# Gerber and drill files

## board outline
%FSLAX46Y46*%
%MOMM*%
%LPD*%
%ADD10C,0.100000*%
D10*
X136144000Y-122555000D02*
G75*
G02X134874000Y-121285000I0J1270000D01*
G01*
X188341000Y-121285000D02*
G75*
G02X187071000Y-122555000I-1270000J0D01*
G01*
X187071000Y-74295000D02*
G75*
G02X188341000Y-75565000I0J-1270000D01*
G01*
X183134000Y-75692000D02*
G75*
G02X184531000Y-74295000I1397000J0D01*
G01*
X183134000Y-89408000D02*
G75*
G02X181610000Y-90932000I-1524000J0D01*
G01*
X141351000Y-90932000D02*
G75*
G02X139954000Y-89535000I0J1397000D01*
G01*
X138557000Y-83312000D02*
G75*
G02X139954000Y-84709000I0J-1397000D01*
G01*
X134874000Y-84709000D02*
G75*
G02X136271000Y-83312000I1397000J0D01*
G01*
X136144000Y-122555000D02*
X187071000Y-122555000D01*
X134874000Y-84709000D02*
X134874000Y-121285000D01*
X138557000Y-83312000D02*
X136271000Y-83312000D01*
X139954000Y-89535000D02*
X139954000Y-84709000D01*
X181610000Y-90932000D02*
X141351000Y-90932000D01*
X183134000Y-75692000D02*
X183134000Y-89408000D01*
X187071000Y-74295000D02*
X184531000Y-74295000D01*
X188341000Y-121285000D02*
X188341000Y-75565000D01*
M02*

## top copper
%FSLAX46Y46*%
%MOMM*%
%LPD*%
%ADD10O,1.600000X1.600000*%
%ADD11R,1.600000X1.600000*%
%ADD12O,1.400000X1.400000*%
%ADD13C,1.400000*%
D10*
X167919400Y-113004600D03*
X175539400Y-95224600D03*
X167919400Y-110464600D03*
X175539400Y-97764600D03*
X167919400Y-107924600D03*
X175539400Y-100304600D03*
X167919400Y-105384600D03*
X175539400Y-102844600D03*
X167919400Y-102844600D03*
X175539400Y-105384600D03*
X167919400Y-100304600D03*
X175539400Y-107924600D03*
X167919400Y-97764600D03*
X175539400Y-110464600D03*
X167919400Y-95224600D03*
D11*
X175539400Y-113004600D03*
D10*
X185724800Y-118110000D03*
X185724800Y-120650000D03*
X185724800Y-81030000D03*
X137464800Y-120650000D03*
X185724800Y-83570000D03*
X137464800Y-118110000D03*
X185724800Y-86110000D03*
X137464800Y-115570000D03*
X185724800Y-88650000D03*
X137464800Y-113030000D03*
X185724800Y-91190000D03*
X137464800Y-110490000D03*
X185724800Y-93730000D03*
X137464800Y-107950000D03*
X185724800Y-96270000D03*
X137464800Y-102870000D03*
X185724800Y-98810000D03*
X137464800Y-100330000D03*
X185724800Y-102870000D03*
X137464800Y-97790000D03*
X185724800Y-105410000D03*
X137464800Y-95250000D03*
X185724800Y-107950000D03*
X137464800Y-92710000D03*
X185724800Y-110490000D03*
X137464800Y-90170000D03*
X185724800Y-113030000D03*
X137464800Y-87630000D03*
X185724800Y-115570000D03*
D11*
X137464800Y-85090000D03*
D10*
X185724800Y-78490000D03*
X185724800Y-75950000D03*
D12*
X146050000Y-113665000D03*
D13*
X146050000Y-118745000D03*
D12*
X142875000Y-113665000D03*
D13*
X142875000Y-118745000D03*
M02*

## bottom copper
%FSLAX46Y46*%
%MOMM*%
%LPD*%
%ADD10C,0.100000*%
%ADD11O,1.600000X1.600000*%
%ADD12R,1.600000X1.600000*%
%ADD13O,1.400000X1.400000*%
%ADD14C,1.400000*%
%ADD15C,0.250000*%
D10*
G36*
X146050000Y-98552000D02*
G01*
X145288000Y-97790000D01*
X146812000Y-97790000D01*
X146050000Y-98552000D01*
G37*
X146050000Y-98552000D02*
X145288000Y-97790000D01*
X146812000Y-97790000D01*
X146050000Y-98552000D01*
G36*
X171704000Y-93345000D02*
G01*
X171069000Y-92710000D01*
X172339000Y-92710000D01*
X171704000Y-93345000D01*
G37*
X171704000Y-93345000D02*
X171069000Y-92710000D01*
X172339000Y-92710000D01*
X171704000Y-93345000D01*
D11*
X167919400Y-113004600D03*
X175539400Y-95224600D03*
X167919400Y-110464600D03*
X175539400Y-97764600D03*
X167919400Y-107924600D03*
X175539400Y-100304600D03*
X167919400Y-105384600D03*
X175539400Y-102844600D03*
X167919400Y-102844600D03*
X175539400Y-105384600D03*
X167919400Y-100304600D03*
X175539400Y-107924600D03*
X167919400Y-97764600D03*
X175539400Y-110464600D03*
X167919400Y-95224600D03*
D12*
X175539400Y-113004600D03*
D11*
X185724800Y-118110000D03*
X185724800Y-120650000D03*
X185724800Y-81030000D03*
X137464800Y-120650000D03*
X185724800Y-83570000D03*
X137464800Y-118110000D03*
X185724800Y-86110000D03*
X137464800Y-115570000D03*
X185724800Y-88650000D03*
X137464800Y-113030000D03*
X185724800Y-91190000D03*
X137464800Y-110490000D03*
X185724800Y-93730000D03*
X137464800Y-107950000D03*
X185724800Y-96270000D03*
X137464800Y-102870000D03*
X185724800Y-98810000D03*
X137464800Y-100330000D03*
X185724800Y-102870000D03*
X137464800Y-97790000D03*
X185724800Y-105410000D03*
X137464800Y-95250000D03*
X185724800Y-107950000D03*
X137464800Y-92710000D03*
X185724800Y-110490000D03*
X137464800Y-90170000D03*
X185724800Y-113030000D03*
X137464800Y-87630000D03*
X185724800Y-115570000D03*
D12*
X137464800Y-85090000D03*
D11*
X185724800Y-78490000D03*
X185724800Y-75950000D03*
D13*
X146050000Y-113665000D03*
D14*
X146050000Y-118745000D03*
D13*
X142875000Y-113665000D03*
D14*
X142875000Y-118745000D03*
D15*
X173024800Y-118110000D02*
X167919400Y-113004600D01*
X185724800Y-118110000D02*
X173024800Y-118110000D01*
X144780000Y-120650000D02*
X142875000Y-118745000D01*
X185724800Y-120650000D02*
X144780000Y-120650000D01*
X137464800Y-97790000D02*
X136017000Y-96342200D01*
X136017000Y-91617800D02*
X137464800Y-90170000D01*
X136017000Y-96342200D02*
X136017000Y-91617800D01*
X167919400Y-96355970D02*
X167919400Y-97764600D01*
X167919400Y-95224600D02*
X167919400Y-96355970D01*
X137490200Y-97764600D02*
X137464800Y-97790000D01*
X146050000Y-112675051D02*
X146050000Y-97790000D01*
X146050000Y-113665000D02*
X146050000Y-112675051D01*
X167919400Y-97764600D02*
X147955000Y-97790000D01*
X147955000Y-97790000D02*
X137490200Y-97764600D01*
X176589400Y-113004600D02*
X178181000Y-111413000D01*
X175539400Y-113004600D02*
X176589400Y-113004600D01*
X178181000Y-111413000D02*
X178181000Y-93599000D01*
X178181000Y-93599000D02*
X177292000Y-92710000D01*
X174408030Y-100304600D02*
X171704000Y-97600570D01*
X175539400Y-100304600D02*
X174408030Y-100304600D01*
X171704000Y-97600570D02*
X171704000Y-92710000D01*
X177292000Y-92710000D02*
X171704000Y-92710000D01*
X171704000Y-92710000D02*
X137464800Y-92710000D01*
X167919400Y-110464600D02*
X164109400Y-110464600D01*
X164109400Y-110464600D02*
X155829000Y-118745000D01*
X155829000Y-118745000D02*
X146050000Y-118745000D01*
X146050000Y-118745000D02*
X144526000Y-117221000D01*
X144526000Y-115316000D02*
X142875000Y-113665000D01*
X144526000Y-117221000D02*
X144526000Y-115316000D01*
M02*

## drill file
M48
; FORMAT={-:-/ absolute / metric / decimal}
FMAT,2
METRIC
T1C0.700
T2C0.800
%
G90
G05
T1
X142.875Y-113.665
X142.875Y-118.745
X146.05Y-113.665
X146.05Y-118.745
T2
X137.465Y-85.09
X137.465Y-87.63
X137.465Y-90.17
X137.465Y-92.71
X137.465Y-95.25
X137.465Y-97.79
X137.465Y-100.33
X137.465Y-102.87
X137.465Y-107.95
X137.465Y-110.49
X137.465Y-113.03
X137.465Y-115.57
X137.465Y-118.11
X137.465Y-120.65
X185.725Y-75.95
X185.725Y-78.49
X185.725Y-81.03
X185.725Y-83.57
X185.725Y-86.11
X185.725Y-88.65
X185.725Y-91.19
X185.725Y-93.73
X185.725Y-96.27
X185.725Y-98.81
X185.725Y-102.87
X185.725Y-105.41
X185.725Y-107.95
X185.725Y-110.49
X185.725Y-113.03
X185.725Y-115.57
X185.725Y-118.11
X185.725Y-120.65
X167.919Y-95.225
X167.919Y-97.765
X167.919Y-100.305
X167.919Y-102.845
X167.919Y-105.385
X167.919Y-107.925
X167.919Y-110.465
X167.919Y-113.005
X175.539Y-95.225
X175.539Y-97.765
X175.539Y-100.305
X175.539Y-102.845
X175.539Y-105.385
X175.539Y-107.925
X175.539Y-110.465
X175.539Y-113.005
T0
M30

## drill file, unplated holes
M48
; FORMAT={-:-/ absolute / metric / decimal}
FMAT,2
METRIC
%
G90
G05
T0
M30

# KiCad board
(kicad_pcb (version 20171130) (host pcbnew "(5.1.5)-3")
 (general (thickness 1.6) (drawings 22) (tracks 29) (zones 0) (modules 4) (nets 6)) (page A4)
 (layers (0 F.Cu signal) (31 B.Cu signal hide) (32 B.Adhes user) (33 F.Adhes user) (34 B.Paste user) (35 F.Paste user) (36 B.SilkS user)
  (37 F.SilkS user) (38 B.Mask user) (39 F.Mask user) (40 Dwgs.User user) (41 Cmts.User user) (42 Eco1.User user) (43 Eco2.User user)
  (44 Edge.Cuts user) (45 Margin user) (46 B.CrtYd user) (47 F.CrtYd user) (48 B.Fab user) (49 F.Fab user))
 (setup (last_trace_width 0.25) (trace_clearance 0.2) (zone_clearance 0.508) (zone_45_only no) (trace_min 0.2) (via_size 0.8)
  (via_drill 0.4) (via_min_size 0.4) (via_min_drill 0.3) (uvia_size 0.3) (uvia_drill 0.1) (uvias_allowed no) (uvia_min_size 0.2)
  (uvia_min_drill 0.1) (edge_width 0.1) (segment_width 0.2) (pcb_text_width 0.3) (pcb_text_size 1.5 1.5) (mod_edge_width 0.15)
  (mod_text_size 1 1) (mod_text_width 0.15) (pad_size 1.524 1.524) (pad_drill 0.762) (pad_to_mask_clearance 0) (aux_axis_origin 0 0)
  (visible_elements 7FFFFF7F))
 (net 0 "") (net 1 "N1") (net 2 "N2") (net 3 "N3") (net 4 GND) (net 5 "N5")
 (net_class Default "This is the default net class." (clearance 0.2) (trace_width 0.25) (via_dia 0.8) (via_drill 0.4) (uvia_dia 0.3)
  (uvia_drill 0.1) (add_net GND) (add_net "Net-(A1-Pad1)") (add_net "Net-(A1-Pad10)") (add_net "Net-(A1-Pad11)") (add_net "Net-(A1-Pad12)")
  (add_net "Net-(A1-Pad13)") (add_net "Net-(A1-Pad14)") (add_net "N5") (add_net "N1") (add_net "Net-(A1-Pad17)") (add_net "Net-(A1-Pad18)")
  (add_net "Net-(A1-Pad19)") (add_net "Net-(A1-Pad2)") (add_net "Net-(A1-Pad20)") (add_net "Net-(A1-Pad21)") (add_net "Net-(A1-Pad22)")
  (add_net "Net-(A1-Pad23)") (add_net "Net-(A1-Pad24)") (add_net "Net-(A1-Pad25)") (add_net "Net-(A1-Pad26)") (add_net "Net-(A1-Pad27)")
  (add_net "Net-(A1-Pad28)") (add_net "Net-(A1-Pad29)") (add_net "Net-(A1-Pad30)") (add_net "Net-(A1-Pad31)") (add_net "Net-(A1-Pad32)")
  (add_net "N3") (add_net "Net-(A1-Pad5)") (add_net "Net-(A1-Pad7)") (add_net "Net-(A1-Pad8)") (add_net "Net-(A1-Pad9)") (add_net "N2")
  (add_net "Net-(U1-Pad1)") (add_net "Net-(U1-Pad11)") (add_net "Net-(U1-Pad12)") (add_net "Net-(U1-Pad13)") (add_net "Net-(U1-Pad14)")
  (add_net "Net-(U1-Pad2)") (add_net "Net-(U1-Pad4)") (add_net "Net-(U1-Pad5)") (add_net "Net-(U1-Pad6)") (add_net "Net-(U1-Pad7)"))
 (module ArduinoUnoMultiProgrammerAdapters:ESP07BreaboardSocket (layer F.Cu) (at 171.704 102.616)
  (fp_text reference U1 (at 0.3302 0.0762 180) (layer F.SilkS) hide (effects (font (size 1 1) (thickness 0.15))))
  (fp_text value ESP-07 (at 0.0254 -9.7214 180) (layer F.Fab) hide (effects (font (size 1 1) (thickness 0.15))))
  (pad 16 thru_hole oval (at -3.7846 10.3886 180) (size 1.6 1.6) (drill 0.8) (layers *.Cu *.Mask) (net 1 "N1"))
  (pad 1 thru_hole oval (at 3.8354 -7.3914 180) (size 1.6 1.6) (drill 0.8) (layers *.Cu *.Mask))
  (pad 15 thru_hole oval (at -3.7846 7.8486 180) (size 1.6 1.6) (drill 0.8) (layers *.Cu *.Mask) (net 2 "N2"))
  (pad 2 thru_hole oval (at 3.8354 -4.8514 180) (size 1.6 1.6) (drill 0.8) (layers *.Cu *.Mask))
  (pad 14 thru_hole oval (at -3.7846 5.3086 180) (size 1.6 1.6) (drill 0.8) (layers *.Cu *.Mask))
  (pad 3 thru_hole oval (at 3.8354 -2.3114 180) (size 1.6 1.6) (drill 0.8) (layers *.Cu *.Mask) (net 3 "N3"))
  (pad 13 thru_hole oval (at -3.7846 2.7686 180) (size 1.6 1.6) (drill 0.8) (layers *.Cu *.Mask))
  (pad 4 thru_hole oval (at 3.8354 0.2286 180) (size 1.6 1.6) (drill 0.8) (layers *.Cu *.Mask))
  (pad 12 thru_hole oval (at -3.7846 0.2286 180) (size 1.6 1.6) (drill 0.8) (layers *.Cu *.Mask))
  (pad 5 thru_hole oval (at 3.8354 2.7686 180) (size 1.6 1.6) (drill 0.8) (layers *.Cu *.Mask))
  (pad 11 thru_hole oval (at -3.7846 -2.3114 180) (size 1.6 1.6) (drill 0.8) (layers *.Cu *.Mask))
  (pad 6 thru_hole oval (at 3.8354 5.3086 180) (size 1.6 1.6) (drill 0.8) (layers *.Cu *.Mask))
  (pad 10 thru_hole oval (at -3.7846 -4.8514 180) (size 1.6 1.6) (drill 0.8) (layers *.Cu *.Mask) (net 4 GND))
  (pad 7 thru_hole oval (at 3.8354 7.8486 180) (size 1.6 1.6) (drill 0.8) (layers *.Cu *.Mask))
  (pad 9 thru_hole oval (at -3.7846 -7.3914 180) (size 1.6 1.6) (drill 0.8) (layers *.Cu *.Mask) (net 4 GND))
  (pad 8 thru_hole rect (at 3.8354 10.3886 270) (size 1.6 1.6) (drill 0.8) (layers *.Cu *.Mask) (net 3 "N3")))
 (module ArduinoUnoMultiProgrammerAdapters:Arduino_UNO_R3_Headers (layer F.Cu) (at 160.274 89.535)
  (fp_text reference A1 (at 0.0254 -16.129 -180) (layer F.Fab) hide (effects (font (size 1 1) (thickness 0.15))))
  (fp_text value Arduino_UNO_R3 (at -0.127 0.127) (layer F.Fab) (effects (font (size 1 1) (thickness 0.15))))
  (pad 16 thru_hole oval (at 25.4508 28.575) (size 1.6 1.6) (drill 0.8) (layers *.Cu *.Mask) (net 1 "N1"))
  (pad 15 thru_hole oval (at 25.4508 31.115) (size 1.6 1.6) (drill 0.8) (layers *.Cu *.Mask) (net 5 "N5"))
  (pad 30 thru_hole oval (at 25.4508 -8.505) (size 1.6 1.6) (drill 0.8) (layers *.Cu *.Mask))
  (pad 14 thru_hole oval (at -22.8092 31.115) (size 1.6 1.6) (drill 0.8) (layers *.Cu *.Mask))
  (pad 29 thru_hole oval (at 25.4508 -5.965) (size 1.6 1.6) (drill 0.8) (layers *.Cu *.Mask))
  (pad 13 thru_hole oval (at -22.8092 28.575) (size 1.6 1.6) (drill 0.8) (layers *.Cu *.Mask))
  (pad 28 thru_hole oval (at 25.4508 -3.425) (size 1.6 1.6) (drill 0.8) (layers *.Cu *.Mask))
  (pad 12 thru_hole oval (at -22.8092 26.035) (size 1.6 1.6) (drill 0.8) (layers *.Cu *.Mask))
  (pad 27 thru_hole oval (at 25.4508 -0.885) (size 1.6 1.6) (drill 0.8) (layers *.Cu *.Mask))
  (pad 11 thru_hole oval (at -22.8092 23.495) (size 1.6 1.6) (drill 0.8) (layers *.Cu *.Mask))
  (pad 26 thru_hole oval (at 25.4508 1.655) (size 1.6 1.6) (drill 0.8) (layers *.Cu *.Mask))
  (pad 10 thru_hole oval (at -22.8092 20.955) (size 1.6 1.6) (drill 0.8) (layers *.Cu *.Mask))
  (pad 25 thru_hole oval (at 25.4508 4.195) (size 1.6 1.6) (drill 0.8) (layers *.Cu *.Mask))
  (pad 9 thru_hole oval (at -22.8092 18.415) (size 1.6 1.6) (drill 0.8) (layers *.Cu *.Mask))
  (pad 24 thru_hole oval (at 25.4508 6.735) (size 1.6 1.6) (drill 0.8) (layers *.Cu *.Mask))
  (pad 8 thru_hole oval (at -22.8092 13.335) (size 1.6 1.6) (drill 0.8) (layers *.Cu *.Mask))
  (pad 23 thru_hole oval (at 25.4508 9.275) (size 1.6 1.6) (drill 0.8) (layers *.Cu *.Mask))
  (pad 7 thru_hole oval (at -22.8092 10.795) (size 1.6 1.6) (drill 0.8) (layers *.Cu *.Mask))
  (pad 22 thru_hole oval (at 25.4508 13.335) (size 1.6 1.6) (drill 0.8) (layers *.Cu *.Mask))
  (pad 6 thru_hole oval (at -22.8092 8.255) (size 1.6 1.6) (drill 0.8) (layers *.Cu *.Mask) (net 4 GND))
  (pad 21 thru_hole oval (at 25.4508 15.875) (size 1.6 1.6) (drill 0.8) (layers *.Cu *.Mask))
  (pad 5 thru_hole oval (at -22.8092 5.715) (size 1.6 1.6) (drill 0.8) (layers *.Cu *.Mask))
  (pad 20 thru_hole oval (at 25.4508 18.415) (size 1.6 1.6) (drill 0.8) (layers *.Cu *.Mask))
  (pad 4 thru_hole oval (at -22.8092 3.175) (size 1.6 1.6) (drill 0.8) (layers *.Cu *.Mask) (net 3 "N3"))
  (pad 19 thru_hole oval (at 25.4508 20.955) (size 1.6 1.6) (drill 0.8) (layers *.Cu *.Mask))
  (pad 3 thru_hole oval (at -22.8092 0.635) (size 1.6 1.6) (drill 0.8) (layers *.Cu *.Mask) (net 4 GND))
  (pad 18 thru_hole oval (at 25.4508 23.495) (size 1.6 1.6) (drill 0.8) (layers *.Cu *.Mask))
  (pad 2 thru_hole oval (at -22.8092 -1.905) (size 1.6 1.6) (drill 0.8) (layers *.Cu *.Mask))
  (pad 17 thru_hole oval (at 25.4508 26.035) (size 1.6 1.6) (drill 0.8) (layers *.Cu *.Mask))
  (pad 1 thru_hole rect (at -22.8092 -4.445) (size 1.6 1.6) (drill 0.8) (layers *.Cu *.Mask))
  (pad 31 thru_hole oval (at 25.4508 -11.045) (size 1.6 1.6) (drill 0.8) (layers *.Cu *.Mask))
  (pad 32 thru_hole oval (at 25.4508 -13.585) (size 1.6 1.6) (drill 0.8) (layers *.Cu *.Mask)))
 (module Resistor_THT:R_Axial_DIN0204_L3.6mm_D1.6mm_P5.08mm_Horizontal (layer F.Cu) (at 146.05 118.745 90)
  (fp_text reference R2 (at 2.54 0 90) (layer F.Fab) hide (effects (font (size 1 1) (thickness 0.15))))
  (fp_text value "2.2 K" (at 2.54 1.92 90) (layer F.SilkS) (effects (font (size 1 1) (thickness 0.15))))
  (pad 2 thru_hole oval (at 5.08 0 90) (size 1.4 1.4) (drill 0.7) (layers *.Cu *.Mask) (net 4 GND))
  (pad 1 thru_hole circle (at 0 0 90) (size 1.4 1.4) (drill 0.7) (layers *.Cu *.Mask) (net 2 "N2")))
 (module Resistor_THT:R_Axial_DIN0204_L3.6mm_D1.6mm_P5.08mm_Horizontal (layer F.Cu) (at 142.875 118.745 90)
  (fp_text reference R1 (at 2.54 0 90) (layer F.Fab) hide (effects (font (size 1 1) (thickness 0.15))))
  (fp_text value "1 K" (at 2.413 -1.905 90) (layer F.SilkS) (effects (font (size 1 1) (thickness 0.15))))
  (pad 2 thru_hole oval (at 5.08 0 90) (size 1.4 1.4) (drill 0.7) (layers *.Cu *.Mask) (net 2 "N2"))
  (pad 1 thru_hole circle (at 0 0 90) (size 1.4 1.4) (drill 0.7) (layers *.Cu *.Mask) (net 5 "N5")))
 (gr_poly (pts (xy 146.05 98.552) (xy 145.288 97.79) (xy 146.812 97.79)) (layer B.Cu) (width 0.1))
 (gr_poly (pts (xy 171.704 93.345) (xy 171.069 92.71) (xy 172.339 92.71)) (layer B.Cu) (width 0.1))
 (gr_arc (start 136.144 121.285) (end 134.874 121.285) (angle -90) (layer Edge.Cuts) (width 0.1))
 (gr_arc (start 187.071 121.285) (end 187.071 122.555) (angle -90) (layer Edge.Cuts) (width 0.1))
 (gr_arc (start 187.071 75.565) (end 188.341 75.565) (angle -90) (layer Edge.Cuts) (width 0.1))
 (gr_arc (start 184.531 75.692) (end 184.531 74.295) (angle -90) (layer Edge.Cuts) (width 0.1))
 (gr_arc (start 181.61 89.408) (end 181.61 90.932) (angle -90) (layer Edge.Cuts) (width 0.1))
 (gr_arc (start 141.351 89.535) (end 139.954 89.535) (angle -90) (layer Edge.Cuts) (width 0.1))
 (gr_arc (start 138.557 84.709) (end 139.954 84.709) (angle -90) (layer Edge.Cuts) (width 0.1))
 (gr_arc (start 136.271 84.709) (end 136.271 83.312) (angle -90) (layer Edge.Cuts) (width 0.1))
 (gr_line (start 136.144 122.555) (end 187.071 122.555) (layer Edge.Cuts) (width 0.1))
 (gr_line (start 134.874 84.709) (end 134.874 121.285) (layer Edge.Cuts) (width 0.1))
 (gr_line (start 138.557 83.312) (end 136.271 83.312) (layer Edge.Cuts) (width 0.1))
 (gr_line (start 139.954 89.535) (end 139.954 84.709) (layer Edge.Cuts) (width 0.1))
 (gr_line (start 181.61 90.932) (end 141.351 90.932) (layer Edge.Cuts) (width 0.1))
 (gr_line (start 183.134 75.692) (end 183.134 89.408) (layer Edge.Cuts) (width 0.1))
 (gr_line (start 187.071 74.295) (end 184.531 74.295) (layer Edge.Cuts) (width 0.1))
 (gr_line (start 188.341 121.285) (end 188.341 75.565) (layer Edge.Cuts) (width 0.1))
 (segment (start 173.0248 118.11) (end 167.9194 113.0046) (width 0.25) (layer B.Cu) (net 1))
 (segment (start 185.7248 118.11) (end 173.0248 118.11) (width 0.25) (layer B.Cu) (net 1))
 (segment (start 144.78 120.65) (end 142.875 118.745) (width 0.25) (layer B.Cu) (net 5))
 (segment (start 185.7248 120.65) (end 144.78 120.65) (width 0.25) (layer B.Cu) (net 5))
 (segment (start 137.4648 97.79) (end 136.017 96.3422) (width 0.25) (layer B.Cu) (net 4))
 (segment (start 136.017 91.6178) (end 137.4648 90.17) (width 0.25) (layer B.Cu) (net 4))
 (segment (start 136.017 96.3422) (end 136.017 91.6178) (width 0.25) (layer B.Cu) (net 4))
 (segment (start 167.9194 96.35597) (end 167.9194 97.7646) (width 0.25) (layer B.Cu) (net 4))
 (segment (start 167.9194 95.2246) (end 167.9194 96.35597) (width 0.25) (layer B.Cu) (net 4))
 (segment (start 137.4902 97.7646) (end 137.4648 97.79) (width 0.25) (layer B.Cu) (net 4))
 (segment (start 146.05 112.675051) (end 146.05 97.79) (width 0.25) (layer B.Cu) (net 4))
 (segment (start 146.05 113.665) (end 146.05 112.675051) (width 0.25) (layer B.Cu) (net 4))
 (segment (start 167.9194 97.7646) (end 147.955 97.79) (width 0.25) (layer B.Cu) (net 4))
 (segment (start 147.955 97.79) (end 137.4902 97.7646) (width 0.25) (layer B.Cu) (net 4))
 (segment (start 176.5894 113.0046) (end 178.181 111.413) (width 0.25) (layer B.Cu) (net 3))
 (segment (start 175.5394 113.0046) (end 176.5894 113.0046) (width 0.25) (layer B.Cu) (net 3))
 (segment (start 178.181 111.413) (end 178.181 93.599) (width 0.25) (layer B.Cu) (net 3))
 (segment (start 178.181 93.599) (end 177.292 92.71) (width 0.25) (layer B.Cu) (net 3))
 (segment (start 174.40803 100.3046) (end 171.704 97.60057) (width 0.25) (layer B.Cu) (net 3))
 (segment (start 175.5394 100.3046) (end 174.40803 100.3046) (width 0.25) (layer B.Cu) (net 3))
 (segment (start 171.704 97.60057) (end 171.704 92.71) (width 0.25) (layer B.Cu) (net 3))
 (segment (start 177.292 92.71) (end 171.704 92.71) (width 0.25) (layer B.Cu) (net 3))
 (segment (start 171.704 92.71) (end 137.4648 92.71) (width 0.25) (layer B.Cu) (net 3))
 (segment (start 167.9194 110.4646) (end 164.1094 110.4646) (width 0.25) (layer B.Cu) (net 2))
 (segment (start 164.1094 110.4646) (end 155.829 118.745) (width 0.25) (layer B.Cu) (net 2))
 (segment (start 155.829 118.745) (end 146.05 118.745) (width 0.25) (layer B.Cu) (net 2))
 (segment (start 146.05 118.745) (end 144.526 117.221) (width 0.25) (layer B.Cu) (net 2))
 (segment (start 144.526 115.316) (end 142.875 113.665) (width 0.25) (layer B.Cu) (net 2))
 (segment (start 144.526 117.221) (end 144.526 115.316) (width 0.25) (layer B.Cu) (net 2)))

